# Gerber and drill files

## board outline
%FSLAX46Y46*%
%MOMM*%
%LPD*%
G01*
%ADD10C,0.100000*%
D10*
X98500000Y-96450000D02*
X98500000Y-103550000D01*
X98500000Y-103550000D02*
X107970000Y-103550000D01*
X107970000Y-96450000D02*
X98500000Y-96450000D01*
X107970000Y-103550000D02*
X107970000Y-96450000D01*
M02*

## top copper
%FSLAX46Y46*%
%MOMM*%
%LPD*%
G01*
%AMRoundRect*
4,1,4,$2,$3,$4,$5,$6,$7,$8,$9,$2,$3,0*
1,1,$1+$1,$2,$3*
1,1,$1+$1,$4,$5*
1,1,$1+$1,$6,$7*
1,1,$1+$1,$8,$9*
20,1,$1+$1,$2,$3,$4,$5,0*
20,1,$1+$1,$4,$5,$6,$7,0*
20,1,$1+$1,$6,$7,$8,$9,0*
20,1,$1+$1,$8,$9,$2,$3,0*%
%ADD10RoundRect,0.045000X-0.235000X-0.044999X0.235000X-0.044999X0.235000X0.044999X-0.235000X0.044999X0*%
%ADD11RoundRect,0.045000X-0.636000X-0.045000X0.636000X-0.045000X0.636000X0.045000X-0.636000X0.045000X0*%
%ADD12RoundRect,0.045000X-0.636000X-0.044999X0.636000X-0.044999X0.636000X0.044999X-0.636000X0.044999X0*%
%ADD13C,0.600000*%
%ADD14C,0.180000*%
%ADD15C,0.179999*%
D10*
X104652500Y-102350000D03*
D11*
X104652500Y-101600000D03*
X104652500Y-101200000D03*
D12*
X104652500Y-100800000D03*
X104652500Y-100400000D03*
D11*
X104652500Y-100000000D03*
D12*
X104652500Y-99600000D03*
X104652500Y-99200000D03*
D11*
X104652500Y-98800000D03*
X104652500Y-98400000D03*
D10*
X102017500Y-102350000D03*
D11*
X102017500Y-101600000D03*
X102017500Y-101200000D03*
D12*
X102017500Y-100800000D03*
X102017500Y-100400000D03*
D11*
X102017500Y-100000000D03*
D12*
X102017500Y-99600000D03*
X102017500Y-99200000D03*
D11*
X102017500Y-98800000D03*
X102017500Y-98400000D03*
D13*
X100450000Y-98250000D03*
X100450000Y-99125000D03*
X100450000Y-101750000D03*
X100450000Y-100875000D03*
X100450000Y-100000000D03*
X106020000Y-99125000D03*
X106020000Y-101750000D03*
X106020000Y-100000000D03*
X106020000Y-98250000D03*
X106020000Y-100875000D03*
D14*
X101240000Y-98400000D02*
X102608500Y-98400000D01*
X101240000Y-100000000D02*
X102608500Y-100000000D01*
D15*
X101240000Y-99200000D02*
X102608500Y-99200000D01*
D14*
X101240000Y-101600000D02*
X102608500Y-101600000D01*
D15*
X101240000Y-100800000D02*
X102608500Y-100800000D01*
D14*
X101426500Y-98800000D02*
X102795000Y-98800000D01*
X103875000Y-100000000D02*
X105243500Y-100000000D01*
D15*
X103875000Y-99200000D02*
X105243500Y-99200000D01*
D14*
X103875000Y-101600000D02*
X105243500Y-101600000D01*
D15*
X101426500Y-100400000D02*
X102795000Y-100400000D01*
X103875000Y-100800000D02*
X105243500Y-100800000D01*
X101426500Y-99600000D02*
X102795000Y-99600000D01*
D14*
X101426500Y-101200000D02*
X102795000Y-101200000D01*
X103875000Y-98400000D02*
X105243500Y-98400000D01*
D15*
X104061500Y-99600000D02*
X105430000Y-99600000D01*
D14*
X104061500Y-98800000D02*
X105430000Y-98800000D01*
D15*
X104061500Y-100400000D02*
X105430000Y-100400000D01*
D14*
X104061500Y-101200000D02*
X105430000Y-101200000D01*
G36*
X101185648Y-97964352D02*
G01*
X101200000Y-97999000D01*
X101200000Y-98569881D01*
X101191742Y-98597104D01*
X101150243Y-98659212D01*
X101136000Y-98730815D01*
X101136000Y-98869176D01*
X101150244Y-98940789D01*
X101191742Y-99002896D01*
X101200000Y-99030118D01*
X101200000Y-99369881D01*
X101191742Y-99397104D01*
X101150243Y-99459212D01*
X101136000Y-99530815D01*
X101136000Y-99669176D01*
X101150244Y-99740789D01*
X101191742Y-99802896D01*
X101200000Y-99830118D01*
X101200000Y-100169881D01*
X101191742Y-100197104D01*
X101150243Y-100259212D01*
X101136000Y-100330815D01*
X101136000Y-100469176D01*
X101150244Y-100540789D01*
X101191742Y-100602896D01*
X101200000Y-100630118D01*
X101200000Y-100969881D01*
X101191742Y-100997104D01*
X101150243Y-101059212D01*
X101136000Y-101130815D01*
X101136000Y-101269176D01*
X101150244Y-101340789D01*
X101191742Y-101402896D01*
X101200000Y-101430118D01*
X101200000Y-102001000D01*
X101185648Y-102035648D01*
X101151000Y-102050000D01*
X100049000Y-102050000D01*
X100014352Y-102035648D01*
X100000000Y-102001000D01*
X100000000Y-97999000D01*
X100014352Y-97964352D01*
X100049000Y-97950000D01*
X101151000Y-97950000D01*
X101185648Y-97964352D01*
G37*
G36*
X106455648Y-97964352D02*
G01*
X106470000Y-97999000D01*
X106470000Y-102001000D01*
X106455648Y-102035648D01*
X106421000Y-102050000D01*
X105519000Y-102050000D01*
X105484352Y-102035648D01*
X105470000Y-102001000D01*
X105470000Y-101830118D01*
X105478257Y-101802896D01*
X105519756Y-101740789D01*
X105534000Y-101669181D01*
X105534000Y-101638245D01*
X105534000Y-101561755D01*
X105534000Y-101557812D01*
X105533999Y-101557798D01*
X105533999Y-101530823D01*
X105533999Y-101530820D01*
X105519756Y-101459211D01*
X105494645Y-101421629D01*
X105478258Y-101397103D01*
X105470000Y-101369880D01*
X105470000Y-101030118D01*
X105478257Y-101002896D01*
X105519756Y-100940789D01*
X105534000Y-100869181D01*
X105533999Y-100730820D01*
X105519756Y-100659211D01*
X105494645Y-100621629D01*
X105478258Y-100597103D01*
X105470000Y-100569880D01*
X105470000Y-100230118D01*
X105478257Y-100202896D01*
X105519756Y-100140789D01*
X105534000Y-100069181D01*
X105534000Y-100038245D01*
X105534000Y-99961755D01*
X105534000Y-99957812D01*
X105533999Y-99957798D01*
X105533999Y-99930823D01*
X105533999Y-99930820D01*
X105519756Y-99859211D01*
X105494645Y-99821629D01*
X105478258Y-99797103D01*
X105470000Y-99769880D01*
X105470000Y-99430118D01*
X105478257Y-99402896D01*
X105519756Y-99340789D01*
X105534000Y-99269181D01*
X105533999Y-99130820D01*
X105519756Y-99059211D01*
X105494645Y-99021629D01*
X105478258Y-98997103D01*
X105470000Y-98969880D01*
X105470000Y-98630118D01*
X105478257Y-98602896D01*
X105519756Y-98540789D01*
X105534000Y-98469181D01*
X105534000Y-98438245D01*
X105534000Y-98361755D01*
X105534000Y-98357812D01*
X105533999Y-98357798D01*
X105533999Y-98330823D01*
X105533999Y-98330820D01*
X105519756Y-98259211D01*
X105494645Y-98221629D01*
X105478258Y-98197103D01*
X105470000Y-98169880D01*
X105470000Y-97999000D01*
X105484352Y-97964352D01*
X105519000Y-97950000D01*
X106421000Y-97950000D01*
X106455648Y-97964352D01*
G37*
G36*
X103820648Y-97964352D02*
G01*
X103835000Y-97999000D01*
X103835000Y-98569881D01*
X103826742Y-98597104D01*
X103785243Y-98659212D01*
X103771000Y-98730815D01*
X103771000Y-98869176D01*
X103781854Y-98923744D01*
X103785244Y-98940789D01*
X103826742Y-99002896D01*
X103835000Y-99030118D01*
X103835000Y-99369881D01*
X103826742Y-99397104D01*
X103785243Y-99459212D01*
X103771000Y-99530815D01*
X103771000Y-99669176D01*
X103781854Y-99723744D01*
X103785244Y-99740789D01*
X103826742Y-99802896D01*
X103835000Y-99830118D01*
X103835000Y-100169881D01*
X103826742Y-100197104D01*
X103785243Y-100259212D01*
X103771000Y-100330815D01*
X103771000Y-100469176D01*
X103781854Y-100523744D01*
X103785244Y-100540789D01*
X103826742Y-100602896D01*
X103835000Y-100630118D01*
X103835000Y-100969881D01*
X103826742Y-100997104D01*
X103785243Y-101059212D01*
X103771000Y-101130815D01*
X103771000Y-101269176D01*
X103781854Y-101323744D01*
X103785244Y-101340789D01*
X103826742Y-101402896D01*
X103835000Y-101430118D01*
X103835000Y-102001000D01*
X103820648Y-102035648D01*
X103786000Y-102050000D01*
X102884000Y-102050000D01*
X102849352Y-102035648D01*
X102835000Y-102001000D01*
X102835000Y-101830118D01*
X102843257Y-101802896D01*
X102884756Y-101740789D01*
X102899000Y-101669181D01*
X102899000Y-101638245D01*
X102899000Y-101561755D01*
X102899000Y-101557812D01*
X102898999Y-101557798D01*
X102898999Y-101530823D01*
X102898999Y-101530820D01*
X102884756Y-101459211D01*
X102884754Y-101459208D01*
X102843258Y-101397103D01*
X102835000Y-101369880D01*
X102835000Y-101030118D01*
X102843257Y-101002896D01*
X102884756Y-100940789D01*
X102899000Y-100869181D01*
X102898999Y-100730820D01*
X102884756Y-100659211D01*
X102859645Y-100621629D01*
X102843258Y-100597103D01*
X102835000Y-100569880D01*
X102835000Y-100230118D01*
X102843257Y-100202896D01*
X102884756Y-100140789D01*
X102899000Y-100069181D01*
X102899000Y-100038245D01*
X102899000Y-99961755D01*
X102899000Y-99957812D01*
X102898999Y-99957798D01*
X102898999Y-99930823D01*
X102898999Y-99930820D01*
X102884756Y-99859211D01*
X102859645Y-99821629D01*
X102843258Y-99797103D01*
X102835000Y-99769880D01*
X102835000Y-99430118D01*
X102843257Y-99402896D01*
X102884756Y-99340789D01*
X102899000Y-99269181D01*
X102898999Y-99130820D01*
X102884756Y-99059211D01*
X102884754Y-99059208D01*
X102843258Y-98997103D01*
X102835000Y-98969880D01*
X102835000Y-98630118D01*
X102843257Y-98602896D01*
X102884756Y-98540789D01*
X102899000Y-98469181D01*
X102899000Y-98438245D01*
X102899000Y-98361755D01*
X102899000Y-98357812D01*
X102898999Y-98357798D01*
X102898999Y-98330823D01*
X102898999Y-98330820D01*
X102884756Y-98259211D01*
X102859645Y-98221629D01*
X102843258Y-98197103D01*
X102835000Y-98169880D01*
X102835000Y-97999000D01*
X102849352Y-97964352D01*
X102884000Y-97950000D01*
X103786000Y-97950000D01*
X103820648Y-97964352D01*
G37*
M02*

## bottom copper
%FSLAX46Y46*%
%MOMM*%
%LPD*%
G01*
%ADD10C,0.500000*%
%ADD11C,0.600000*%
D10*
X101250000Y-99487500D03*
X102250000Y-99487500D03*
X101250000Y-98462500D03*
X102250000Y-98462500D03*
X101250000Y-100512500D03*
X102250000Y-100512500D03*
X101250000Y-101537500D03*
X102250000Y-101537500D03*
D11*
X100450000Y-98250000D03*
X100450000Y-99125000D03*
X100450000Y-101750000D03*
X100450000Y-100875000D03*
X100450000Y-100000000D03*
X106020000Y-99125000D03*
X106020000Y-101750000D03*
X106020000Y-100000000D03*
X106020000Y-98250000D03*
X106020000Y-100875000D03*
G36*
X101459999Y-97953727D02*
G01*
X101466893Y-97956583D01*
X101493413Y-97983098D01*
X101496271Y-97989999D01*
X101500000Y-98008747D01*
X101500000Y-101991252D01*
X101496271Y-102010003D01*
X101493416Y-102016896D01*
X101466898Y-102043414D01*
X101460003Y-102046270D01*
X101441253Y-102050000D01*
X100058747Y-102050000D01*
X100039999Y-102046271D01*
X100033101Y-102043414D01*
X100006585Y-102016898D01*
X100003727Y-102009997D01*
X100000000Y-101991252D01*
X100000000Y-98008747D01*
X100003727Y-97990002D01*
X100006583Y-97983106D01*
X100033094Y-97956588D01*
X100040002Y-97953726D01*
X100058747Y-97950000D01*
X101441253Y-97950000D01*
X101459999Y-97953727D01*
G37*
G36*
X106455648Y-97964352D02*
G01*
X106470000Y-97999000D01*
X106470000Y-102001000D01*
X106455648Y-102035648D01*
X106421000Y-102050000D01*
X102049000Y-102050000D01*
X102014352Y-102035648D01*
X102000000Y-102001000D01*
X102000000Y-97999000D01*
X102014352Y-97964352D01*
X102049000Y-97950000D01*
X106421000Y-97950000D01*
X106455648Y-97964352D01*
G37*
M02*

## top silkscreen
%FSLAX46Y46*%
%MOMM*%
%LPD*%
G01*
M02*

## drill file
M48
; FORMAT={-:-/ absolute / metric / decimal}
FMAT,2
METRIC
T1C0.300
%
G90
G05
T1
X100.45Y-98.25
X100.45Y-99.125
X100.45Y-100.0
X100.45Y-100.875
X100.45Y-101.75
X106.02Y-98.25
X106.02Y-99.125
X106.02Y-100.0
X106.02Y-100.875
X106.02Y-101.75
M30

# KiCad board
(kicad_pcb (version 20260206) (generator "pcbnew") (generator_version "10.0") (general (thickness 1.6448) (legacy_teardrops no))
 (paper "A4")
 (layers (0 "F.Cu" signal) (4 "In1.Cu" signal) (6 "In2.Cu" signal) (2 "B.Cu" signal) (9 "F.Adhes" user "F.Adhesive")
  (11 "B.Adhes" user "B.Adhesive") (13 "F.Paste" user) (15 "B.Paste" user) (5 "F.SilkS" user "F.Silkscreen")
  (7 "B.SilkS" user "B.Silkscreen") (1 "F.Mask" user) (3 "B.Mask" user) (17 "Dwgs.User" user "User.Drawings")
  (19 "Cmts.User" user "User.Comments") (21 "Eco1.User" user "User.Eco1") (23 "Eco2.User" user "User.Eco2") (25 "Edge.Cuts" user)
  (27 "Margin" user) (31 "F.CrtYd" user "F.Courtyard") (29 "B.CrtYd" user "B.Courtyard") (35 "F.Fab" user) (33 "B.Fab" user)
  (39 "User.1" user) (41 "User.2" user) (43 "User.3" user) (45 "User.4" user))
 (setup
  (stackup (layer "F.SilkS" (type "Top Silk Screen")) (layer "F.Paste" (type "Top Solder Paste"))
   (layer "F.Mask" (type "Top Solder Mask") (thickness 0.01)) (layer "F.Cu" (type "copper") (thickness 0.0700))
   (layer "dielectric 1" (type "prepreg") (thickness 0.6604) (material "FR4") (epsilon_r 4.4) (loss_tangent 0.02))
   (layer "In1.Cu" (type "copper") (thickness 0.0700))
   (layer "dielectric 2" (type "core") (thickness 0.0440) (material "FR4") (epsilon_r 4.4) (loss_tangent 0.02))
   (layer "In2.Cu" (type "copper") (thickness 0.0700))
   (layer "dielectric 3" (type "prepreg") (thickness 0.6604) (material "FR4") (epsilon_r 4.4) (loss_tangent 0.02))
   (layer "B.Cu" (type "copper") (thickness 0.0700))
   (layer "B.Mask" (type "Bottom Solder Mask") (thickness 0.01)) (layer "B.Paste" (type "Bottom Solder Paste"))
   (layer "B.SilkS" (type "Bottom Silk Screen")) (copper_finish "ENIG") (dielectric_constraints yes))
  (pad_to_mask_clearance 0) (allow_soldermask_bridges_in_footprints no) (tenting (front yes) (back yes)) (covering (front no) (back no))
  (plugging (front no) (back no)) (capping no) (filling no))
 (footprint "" (layer "F.Cu") (at 0 0)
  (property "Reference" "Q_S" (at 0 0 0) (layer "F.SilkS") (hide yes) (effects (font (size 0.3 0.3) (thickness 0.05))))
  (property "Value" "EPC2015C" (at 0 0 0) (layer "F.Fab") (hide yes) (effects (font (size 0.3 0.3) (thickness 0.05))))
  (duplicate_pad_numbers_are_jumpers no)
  (pad "1" smd roundrect (at 104.6525 102.35) (size 0.56 0.179999) (layers "F.Cu" "F.Mask" "F.Paste") (roundrect_rratio 0.25) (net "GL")
   (thermal_bridge_angle 45))
  (pad "3" smd roundrect (at 104.6525 101.6) (size 1.362 0.18) (layers "F.Cu" "F.Mask" "F.Paste") (roundrect_rratio 0.25) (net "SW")
   (thermal_bridge_angle 45))
  (pad "4" smd roundrect (at 104.6525 101.2) (size 1.362 0.18) (layers "F.Cu" "F.Mask" "F.Paste") (roundrect_rratio 0.25) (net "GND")
   (thermal_bridge_angle 45))
  (pad "5" smd roundrect (at 104.6525 100.8) (size 1.362 0.179999) (layers "F.Cu" "F.Mask" "F.Paste") (roundrect_rratio 0.25) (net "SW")
   (thermal_bridge_angle 45))
  (pad "6" smd roundrect (at 104.6525 100.4) (size 1.362 0.179999) (layers "F.Cu" "F.Mask" "F.Paste") (roundrect_rratio 0.25) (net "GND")
   (thermal_bridge_angle 45))
  (pad "7" smd roundrect (at 104.6525 100) (size 1.362 0.18) (layers "F.Cu" "F.Mask" "F.Paste") (roundrect_rratio 0.25) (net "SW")
   (thermal_bridge_angle 45))
  (pad "8" smd roundrect (at 104.6525 99.6) (size 1.362 0.179999) (layers "F.Cu" "F.Mask" "F.Paste") (roundrect_rratio 0.25) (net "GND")
   (thermal_bridge_angle 45))
  (pad "9" smd roundrect (at 104.6525 99.2) (size 1.362 0.179999) (layers "F.Cu" "F.Mask" "F.Paste") (roundrect_rratio 0.25) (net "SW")
   (thermal_bridge_angle 45))
  (pad "10" smd roundrect (at 104.6525 98.8) (size 1.362 0.18) (layers "F.Cu" "F.Mask" "F.Paste") (roundrect_rratio 0.25) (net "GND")
   (thermal_bridge_angle 45))
  (pad "11" smd roundrect (at 104.6525 98.4) (size 1.362 0.18) (layers "F.Cu" "F.Mask" "F.Paste") (roundrect_rratio 0.25) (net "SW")
   (thermal_bridge_angle 45)))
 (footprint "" (layer "F.Cu") (at 0 0)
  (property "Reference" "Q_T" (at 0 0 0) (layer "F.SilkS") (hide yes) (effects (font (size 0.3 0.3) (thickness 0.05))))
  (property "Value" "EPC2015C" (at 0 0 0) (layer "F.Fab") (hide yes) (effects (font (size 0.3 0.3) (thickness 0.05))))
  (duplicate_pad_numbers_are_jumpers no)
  (pad "1" smd roundrect (at 102.0175 102.35) (size 0.56 0.179999) (layers "F.Cu" "F.Mask" "F.Paste") (roundrect_rratio 0.25) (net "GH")
   (thermal_bridge_angle 45))
  (pad "3" smd roundrect (at 102.0175 101.6) (size 1.362 0.18) (layers "F.Cu" "F.Mask" "F.Paste") (roundrect_rratio 0.25) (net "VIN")
   (thermal_bridge_angle 45))
  (pad "4" smd roundrect (at 102.0175 101.2) (size 1.362 0.18) (layers "F.Cu" "F.Mask" "F.Paste") (roundrect_rratio 0.25) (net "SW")
   (thermal_bridge_angle 45))
  (pad "5" smd roundrect (at 102.0175 100.8) (size 1.362 0.179999) (layers "F.Cu" "F.Mask" "F.Paste") (roundrect_rratio 0.25) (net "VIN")
   (thermal_bridge_angle 45))
  (pad "6" smd roundrect (at 102.0175 100.4) (size 1.362 0.179999) (layers "F.Cu" "F.Mask" "F.Paste") (roundrect_rratio 0.25) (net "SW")
   (thermal_bridge_angle 45))
  (pad "7" smd roundrect (at 102.0175 100) (size 1.362 0.18) (layers "F.Cu" "F.Mask" "F.Paste") (roundrect_rratio 0.25) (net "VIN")
   (thermal_bridge_angle 45))
  (pad "8" smd roundrect (at 102.0175 99.6) (size 1.362 0.179999) (layers "F.Cu" "F.Mask" "F.Paste") (roundrect_rratio 0.25) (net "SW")
   (thermal_bridge_angle 45))
  (pad "9" smd roundrect (at 102.0175 99.2) (size 1.362 0.179999) (layers "F.Cu" "F.Mask" "F.Paste") (roundrect_rratio 0.25) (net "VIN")
   (thermal_bridge_angle 45))
  (pad "10" smd roundrect (at 102.0175 98.8) (size 1.362 0.18) (layers "F.Cu" "F.Mask" "F.Paste") (roundrect_rratio 0.25) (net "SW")
   (thermal_bridge_angle 45))
  (pad "11" smd roundrect (at 102.0175 98.4) (size 1.362 0.18) (layers "F.Cu" "F.Mask" "F.Paste") (roundrect_rratio 0.25) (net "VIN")
   (thermal_bridge_angle 45)))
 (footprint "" (layer "B.Cu") (at 101.75 99.4875)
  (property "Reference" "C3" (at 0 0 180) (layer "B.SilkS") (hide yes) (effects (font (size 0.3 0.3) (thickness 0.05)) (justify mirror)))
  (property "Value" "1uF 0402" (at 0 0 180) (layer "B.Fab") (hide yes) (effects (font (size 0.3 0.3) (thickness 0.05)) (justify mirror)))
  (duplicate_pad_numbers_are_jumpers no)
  (pad "1" smd circle (at -0.5 0) (size 0.5 0.5) (layers "B.Cu" "B.Mask" "B.Paste") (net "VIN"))
  (pad "2" smd circle (at 0.5 0) (size 0.5 0.5) (layers "B.Cu" "B.Mask" "B.Paste") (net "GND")))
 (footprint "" (layer "B.Cu") (at 101.75 98.4625)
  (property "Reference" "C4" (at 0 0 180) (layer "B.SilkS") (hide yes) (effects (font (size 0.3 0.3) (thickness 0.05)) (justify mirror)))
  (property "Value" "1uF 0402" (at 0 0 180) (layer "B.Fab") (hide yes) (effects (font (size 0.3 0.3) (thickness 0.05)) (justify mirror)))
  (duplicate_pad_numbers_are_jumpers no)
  (pad "1" smd circle (at -0.5 0) (size 0.5 0.5) (layers "B.Cu" "B.Mask" "B.Paste") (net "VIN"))
  (pad "2" smd circle (at 0.5 0) (size 0.5 0.5) (layers "B.Cu" "B.Mask" "B.Paste") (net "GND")))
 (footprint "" (layer "B.Cu") (at 101.75 100.5125)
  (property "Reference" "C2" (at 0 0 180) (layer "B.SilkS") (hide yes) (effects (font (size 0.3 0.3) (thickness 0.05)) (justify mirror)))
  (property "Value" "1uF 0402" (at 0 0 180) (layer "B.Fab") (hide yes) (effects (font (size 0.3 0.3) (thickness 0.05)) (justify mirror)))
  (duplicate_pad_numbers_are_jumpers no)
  (pad "1" smd circle (at -0.5 0) (size 0.5 0.5) (layers "B.Cu" "B.Mask" "B.Paste") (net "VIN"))
  (pad "2" smd circle (at 0.5 0) (size 0.5 0.5) (layers "B.Cu" "B.Mask" "B.Paste") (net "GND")))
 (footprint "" (layer "B.Cu") (at 101.75 101.5375)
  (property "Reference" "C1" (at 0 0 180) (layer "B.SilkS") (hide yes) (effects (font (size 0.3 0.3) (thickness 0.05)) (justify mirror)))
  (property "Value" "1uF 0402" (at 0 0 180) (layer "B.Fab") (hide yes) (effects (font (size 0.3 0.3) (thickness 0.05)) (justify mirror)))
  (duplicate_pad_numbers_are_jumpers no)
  (pad "1" smd circle (at -0.5 0) (size 0.5 0.5) (layers "B.Cu" "B.Mask" "B.Paste") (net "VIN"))
  (pad "2" smd circle (at 0.5 0) (size 0.5 0.5) (layers "B.Cu" "B.Mask" "B.Paste") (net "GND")))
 (gr_line (start 98.5 96.45) (end 98.5 103.55) (stroke (width 0.1) (type default)) (layer "Edge.Cuts"))
 (gr_line (start 98.5 103.55) (end 107.97 103.55) (stroke (width 0.1) (type default)) (layer "Edge.Cuts"))
 (gr_line (start 107.97 96.45) (end 98.5 96.45) (stroke (width 0.1) (type default)) (layer "Edge.Cuts"))
 (gr_line (start 107.97 103.55) (end 107.97 96.45) (stroke (width 0.1) (type default)) (layer "Edge.Cuts"))
 (segment (start 101.24 98.4) (end 102.6085 98.4) (width 0.18) (layer "F.Cu") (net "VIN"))
 (segment (start 101.24 100) (end 102.6085 100) (width 0.18) (layer "F.Cu") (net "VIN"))
 (segment (start 101.24 99.2) (end 102.6085 99.2) (width 0.179999) (layer "F.Cu") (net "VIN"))
 (segment (start 101.24 101.6) (end 102.6085 101.6) (width 0.18) (layer "F.Cu") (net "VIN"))
 (segment (start 101.24 100.8) (end 102.6085 100.8) (width 0.179999) (layer "F.Cu") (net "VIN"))
 (via (at 100.45 98.25) (size 0.6) (drill 0.3) (layers "F.Cu" "B.Cu") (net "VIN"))
 (via (at 100.45 99.125) (size 0.6) (drill 0.3) (layers "F.Cu" "B.Cu") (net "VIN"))
 (via (at 100.45 101.75) (size 0.6) (drill 0.3) (layers "F.Cu" "B.Cu") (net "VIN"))
 (via (at 100.45 100.875) (size 0.6) (drill 0.3) (layers "F.Cu" "B.Cu") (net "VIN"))
 (via (at 100.45 100) (size 0.6) (drill 0.3) (layers "F.Cu" "B.Cu") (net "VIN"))
 (segment (start 101.4265 98.8) (end 102.795 98.8) (width 0.18) (layer "F.Cu") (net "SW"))
 (segment (start 103.875 100) (end 105.2435 100) (width 0.18) (layer "F.Cu") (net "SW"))
 (segment (start 103.875 99.2) (end 105.2435 99.2) (width 0.179999) (layer "F.Cu") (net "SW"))
 (segment (start 103.875 101.6) (end 105.2435 101.6) (width 0.18) (layer "F.Cu") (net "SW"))
 (segment (start 101.4265 100.4) (end 102.795 100.4) (width 0.179999) (layer "F.Cu") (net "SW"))
 (segment (start 103.875 100.8) (end 105.2435 100.8) (width 0.179999) (layer "F.Cu") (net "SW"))
 (segment (start 101.4265 99.6) (end 102.795 99.6) (width 0.179999) (layer "F.Cu") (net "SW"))
 (segment (start 101.4265 101.2) (end 102.795 101.2) (width 0.18) (layer "F.Cu") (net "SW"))
 (segment (start 103.875 98.4) (end 105.2435 98.4) (width 0.18) (layer "F.Cu") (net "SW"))
 (segment (start 104.0615 99.6) (end 105.43 99.6) (width 0.179999) (layer "F.Cu") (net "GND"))
 (segment (start 104.0615 98.8) (end 105.43 98.8) (width 0.18) (layer "F.Cu") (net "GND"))
 (segment (start 104.0615 100.4) (end 105.43 100.4) (width 0.179999) (layer "F.Cu") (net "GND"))
 (segment (start 104.0615 101.2) (end 105.43 101.2) (width 0.18) (layer "F.Cu") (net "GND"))
 (via (at 106.02 99.125) (size 0.6) (drill 0.3) (layers "F.Cu" "B.Cu") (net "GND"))
 (via (at 106.02 101.75) (size 0.6) (drill 0.3) (layers "F.Cu" "B.Cu") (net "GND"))
 (via (at 106.02 100) (size 0.6) (drill 0.3) (layers "F.Cu" "B.Cu") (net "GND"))
 (via (at 106.02 98.25) (size 0.6) (drill 0.3) (layers "F.Cu" "B.Cu") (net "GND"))
 (via (at 106.02 100.875) (size 0.6) (drill 0.3) (layers "F.Cu" "B.Cu") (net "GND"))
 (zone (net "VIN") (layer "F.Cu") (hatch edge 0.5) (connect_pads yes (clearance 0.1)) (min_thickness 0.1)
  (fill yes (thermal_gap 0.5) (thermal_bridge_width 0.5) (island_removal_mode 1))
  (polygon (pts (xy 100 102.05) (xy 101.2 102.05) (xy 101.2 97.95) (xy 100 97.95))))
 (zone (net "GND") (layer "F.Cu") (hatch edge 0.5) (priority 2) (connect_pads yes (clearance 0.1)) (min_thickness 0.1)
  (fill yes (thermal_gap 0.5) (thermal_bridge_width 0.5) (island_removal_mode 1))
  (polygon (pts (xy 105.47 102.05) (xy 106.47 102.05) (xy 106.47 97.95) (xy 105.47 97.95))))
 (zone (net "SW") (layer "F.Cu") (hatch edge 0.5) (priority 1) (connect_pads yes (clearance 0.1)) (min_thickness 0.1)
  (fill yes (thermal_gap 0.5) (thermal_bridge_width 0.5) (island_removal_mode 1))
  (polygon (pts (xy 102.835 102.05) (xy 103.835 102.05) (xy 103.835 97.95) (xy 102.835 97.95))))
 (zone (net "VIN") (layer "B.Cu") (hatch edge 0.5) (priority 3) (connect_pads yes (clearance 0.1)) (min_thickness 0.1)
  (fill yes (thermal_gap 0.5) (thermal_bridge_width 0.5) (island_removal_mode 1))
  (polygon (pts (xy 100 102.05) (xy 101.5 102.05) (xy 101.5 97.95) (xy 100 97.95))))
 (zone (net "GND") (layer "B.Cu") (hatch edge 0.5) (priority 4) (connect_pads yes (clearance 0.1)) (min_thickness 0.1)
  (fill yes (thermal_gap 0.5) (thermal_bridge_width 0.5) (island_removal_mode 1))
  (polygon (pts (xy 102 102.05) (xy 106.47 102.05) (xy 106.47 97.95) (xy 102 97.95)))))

